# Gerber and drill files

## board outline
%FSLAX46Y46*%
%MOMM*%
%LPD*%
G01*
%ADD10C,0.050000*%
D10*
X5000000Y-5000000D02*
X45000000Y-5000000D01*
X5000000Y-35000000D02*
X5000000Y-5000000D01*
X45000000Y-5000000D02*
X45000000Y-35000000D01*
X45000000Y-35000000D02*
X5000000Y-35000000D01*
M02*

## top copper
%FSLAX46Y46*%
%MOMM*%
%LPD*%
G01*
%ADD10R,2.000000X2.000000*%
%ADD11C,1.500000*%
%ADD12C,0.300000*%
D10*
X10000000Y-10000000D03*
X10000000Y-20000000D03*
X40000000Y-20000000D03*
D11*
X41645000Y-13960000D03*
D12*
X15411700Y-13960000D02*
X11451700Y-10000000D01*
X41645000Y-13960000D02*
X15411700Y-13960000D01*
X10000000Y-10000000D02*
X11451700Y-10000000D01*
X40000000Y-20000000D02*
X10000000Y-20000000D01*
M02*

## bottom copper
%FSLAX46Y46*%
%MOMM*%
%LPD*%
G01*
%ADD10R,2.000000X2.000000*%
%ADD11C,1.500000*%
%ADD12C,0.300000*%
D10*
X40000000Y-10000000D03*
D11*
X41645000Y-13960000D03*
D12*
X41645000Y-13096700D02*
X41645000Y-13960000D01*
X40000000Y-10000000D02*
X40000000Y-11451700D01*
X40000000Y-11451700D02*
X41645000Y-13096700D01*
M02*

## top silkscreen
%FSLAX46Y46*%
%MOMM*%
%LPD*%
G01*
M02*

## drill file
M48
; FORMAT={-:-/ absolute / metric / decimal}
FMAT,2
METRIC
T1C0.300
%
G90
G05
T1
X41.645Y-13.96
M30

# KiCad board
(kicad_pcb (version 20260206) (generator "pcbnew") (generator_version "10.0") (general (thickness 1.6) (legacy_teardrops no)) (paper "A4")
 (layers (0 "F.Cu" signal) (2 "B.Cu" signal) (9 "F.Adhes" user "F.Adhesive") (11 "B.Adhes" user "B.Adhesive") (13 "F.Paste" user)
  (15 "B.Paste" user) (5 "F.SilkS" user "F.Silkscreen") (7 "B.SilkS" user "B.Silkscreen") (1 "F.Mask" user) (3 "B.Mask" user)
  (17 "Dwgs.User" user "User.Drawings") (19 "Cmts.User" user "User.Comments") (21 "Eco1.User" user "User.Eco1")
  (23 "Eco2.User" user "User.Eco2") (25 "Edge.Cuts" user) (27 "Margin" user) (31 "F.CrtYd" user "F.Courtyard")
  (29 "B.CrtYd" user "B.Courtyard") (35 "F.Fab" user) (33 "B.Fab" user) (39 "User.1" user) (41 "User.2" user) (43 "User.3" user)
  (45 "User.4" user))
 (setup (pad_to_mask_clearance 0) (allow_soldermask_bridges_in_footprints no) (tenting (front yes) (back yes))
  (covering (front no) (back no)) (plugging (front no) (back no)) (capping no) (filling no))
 (gr_line (start 5 5) (end 45 5) (stroke (width 0.05) (type default)) (layer "Edge.Cuts"))
 (gr_line (start 5 35) (end 5 5) (stroke (width 0.05) (type default)) (layer "Edge.Cuts"))
 (gr_line (start 45 5) (end 45 35) (stroke (width 0.05) (type default)) (layer "Edge.Cuts"))
 (gr_line (start 45 35) (end 5 35) (stroke (width 0.05) (type default)) (layer "Edge.Cuts"))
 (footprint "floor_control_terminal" (layer "F.Cu") (at 10 10)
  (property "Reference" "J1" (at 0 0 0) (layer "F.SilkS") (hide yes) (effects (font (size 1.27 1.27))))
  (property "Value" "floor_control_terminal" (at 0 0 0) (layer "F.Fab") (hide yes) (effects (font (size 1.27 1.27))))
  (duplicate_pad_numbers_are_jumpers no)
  (pad "1" smd rect (at 0 0) (size 2 2) (layers "F.Cu" "F.Paste" "F.Mask") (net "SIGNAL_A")))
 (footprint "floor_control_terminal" (layer "B.Cu") (at 40 10)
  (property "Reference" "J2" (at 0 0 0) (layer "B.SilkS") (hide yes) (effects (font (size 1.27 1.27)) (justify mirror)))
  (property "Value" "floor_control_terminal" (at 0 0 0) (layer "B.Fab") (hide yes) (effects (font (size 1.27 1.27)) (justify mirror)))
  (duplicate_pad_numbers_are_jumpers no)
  (pad "1" smd rect (at 0 0) (size 2 2) (layers "B.Cu" "B.Paste" "B.Mask") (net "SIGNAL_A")))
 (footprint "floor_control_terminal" (layer "F.Cu") (at 10 20)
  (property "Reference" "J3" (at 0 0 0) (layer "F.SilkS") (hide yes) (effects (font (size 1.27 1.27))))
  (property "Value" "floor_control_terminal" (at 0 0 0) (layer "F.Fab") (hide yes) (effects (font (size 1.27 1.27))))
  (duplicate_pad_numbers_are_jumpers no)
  (pad "1" smd rect (at 0 0) (size 2 2) (layers "F.Cu" "F.Paste" "F.Mask") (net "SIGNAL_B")))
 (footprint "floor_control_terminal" (layer "F.Cu") (at 40 20)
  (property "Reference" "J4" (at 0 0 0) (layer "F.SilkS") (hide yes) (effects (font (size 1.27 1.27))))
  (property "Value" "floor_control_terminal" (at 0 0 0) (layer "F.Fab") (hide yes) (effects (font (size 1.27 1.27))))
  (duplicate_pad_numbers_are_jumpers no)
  (pad "1" smd rect (at 0 0) (size 2 2) (layers "F.Cu" "F.Paste" "F.Mask") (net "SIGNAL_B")))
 (segment (start 15.4117 13.96) (end 11.4517 10) (width 0.3) (layer "F.Cu") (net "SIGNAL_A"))
 (segment (start 41.645 13.96) (end 15.4117 13.96) (width 0.3) (layer "F.Cu") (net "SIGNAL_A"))
 (segment (start 10 10) (end 11.4517 10) (width 0.3) (layer "F.Cu") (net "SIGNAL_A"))
 (via (at 41.645 13.96) (size 1.5) (drill 0.3) (layers "F.Cu" "B.Cu") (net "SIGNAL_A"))
 (segment (start 41.645 13.0967) (end 41.645 13.96) (width 0.3) (layer "B.Cu") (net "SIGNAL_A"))
 (segment (start 40 10) (end 40 11.4517) (width 0.3) (layer "B.Cu") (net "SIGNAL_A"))
 (segment (start 40 11.4517) (end 41.645 13.0967) (width 0.3) (layer "B.Cu") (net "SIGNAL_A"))
 (segment (start 40 20) (end 10 20) (width 0.3) (layer "F.Cu") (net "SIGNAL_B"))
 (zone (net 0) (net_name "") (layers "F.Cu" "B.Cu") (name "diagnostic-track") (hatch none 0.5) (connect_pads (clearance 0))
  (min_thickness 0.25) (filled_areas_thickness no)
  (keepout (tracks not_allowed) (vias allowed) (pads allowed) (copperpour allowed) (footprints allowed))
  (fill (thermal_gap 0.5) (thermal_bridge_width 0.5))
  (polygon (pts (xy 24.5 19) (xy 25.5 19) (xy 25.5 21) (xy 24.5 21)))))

